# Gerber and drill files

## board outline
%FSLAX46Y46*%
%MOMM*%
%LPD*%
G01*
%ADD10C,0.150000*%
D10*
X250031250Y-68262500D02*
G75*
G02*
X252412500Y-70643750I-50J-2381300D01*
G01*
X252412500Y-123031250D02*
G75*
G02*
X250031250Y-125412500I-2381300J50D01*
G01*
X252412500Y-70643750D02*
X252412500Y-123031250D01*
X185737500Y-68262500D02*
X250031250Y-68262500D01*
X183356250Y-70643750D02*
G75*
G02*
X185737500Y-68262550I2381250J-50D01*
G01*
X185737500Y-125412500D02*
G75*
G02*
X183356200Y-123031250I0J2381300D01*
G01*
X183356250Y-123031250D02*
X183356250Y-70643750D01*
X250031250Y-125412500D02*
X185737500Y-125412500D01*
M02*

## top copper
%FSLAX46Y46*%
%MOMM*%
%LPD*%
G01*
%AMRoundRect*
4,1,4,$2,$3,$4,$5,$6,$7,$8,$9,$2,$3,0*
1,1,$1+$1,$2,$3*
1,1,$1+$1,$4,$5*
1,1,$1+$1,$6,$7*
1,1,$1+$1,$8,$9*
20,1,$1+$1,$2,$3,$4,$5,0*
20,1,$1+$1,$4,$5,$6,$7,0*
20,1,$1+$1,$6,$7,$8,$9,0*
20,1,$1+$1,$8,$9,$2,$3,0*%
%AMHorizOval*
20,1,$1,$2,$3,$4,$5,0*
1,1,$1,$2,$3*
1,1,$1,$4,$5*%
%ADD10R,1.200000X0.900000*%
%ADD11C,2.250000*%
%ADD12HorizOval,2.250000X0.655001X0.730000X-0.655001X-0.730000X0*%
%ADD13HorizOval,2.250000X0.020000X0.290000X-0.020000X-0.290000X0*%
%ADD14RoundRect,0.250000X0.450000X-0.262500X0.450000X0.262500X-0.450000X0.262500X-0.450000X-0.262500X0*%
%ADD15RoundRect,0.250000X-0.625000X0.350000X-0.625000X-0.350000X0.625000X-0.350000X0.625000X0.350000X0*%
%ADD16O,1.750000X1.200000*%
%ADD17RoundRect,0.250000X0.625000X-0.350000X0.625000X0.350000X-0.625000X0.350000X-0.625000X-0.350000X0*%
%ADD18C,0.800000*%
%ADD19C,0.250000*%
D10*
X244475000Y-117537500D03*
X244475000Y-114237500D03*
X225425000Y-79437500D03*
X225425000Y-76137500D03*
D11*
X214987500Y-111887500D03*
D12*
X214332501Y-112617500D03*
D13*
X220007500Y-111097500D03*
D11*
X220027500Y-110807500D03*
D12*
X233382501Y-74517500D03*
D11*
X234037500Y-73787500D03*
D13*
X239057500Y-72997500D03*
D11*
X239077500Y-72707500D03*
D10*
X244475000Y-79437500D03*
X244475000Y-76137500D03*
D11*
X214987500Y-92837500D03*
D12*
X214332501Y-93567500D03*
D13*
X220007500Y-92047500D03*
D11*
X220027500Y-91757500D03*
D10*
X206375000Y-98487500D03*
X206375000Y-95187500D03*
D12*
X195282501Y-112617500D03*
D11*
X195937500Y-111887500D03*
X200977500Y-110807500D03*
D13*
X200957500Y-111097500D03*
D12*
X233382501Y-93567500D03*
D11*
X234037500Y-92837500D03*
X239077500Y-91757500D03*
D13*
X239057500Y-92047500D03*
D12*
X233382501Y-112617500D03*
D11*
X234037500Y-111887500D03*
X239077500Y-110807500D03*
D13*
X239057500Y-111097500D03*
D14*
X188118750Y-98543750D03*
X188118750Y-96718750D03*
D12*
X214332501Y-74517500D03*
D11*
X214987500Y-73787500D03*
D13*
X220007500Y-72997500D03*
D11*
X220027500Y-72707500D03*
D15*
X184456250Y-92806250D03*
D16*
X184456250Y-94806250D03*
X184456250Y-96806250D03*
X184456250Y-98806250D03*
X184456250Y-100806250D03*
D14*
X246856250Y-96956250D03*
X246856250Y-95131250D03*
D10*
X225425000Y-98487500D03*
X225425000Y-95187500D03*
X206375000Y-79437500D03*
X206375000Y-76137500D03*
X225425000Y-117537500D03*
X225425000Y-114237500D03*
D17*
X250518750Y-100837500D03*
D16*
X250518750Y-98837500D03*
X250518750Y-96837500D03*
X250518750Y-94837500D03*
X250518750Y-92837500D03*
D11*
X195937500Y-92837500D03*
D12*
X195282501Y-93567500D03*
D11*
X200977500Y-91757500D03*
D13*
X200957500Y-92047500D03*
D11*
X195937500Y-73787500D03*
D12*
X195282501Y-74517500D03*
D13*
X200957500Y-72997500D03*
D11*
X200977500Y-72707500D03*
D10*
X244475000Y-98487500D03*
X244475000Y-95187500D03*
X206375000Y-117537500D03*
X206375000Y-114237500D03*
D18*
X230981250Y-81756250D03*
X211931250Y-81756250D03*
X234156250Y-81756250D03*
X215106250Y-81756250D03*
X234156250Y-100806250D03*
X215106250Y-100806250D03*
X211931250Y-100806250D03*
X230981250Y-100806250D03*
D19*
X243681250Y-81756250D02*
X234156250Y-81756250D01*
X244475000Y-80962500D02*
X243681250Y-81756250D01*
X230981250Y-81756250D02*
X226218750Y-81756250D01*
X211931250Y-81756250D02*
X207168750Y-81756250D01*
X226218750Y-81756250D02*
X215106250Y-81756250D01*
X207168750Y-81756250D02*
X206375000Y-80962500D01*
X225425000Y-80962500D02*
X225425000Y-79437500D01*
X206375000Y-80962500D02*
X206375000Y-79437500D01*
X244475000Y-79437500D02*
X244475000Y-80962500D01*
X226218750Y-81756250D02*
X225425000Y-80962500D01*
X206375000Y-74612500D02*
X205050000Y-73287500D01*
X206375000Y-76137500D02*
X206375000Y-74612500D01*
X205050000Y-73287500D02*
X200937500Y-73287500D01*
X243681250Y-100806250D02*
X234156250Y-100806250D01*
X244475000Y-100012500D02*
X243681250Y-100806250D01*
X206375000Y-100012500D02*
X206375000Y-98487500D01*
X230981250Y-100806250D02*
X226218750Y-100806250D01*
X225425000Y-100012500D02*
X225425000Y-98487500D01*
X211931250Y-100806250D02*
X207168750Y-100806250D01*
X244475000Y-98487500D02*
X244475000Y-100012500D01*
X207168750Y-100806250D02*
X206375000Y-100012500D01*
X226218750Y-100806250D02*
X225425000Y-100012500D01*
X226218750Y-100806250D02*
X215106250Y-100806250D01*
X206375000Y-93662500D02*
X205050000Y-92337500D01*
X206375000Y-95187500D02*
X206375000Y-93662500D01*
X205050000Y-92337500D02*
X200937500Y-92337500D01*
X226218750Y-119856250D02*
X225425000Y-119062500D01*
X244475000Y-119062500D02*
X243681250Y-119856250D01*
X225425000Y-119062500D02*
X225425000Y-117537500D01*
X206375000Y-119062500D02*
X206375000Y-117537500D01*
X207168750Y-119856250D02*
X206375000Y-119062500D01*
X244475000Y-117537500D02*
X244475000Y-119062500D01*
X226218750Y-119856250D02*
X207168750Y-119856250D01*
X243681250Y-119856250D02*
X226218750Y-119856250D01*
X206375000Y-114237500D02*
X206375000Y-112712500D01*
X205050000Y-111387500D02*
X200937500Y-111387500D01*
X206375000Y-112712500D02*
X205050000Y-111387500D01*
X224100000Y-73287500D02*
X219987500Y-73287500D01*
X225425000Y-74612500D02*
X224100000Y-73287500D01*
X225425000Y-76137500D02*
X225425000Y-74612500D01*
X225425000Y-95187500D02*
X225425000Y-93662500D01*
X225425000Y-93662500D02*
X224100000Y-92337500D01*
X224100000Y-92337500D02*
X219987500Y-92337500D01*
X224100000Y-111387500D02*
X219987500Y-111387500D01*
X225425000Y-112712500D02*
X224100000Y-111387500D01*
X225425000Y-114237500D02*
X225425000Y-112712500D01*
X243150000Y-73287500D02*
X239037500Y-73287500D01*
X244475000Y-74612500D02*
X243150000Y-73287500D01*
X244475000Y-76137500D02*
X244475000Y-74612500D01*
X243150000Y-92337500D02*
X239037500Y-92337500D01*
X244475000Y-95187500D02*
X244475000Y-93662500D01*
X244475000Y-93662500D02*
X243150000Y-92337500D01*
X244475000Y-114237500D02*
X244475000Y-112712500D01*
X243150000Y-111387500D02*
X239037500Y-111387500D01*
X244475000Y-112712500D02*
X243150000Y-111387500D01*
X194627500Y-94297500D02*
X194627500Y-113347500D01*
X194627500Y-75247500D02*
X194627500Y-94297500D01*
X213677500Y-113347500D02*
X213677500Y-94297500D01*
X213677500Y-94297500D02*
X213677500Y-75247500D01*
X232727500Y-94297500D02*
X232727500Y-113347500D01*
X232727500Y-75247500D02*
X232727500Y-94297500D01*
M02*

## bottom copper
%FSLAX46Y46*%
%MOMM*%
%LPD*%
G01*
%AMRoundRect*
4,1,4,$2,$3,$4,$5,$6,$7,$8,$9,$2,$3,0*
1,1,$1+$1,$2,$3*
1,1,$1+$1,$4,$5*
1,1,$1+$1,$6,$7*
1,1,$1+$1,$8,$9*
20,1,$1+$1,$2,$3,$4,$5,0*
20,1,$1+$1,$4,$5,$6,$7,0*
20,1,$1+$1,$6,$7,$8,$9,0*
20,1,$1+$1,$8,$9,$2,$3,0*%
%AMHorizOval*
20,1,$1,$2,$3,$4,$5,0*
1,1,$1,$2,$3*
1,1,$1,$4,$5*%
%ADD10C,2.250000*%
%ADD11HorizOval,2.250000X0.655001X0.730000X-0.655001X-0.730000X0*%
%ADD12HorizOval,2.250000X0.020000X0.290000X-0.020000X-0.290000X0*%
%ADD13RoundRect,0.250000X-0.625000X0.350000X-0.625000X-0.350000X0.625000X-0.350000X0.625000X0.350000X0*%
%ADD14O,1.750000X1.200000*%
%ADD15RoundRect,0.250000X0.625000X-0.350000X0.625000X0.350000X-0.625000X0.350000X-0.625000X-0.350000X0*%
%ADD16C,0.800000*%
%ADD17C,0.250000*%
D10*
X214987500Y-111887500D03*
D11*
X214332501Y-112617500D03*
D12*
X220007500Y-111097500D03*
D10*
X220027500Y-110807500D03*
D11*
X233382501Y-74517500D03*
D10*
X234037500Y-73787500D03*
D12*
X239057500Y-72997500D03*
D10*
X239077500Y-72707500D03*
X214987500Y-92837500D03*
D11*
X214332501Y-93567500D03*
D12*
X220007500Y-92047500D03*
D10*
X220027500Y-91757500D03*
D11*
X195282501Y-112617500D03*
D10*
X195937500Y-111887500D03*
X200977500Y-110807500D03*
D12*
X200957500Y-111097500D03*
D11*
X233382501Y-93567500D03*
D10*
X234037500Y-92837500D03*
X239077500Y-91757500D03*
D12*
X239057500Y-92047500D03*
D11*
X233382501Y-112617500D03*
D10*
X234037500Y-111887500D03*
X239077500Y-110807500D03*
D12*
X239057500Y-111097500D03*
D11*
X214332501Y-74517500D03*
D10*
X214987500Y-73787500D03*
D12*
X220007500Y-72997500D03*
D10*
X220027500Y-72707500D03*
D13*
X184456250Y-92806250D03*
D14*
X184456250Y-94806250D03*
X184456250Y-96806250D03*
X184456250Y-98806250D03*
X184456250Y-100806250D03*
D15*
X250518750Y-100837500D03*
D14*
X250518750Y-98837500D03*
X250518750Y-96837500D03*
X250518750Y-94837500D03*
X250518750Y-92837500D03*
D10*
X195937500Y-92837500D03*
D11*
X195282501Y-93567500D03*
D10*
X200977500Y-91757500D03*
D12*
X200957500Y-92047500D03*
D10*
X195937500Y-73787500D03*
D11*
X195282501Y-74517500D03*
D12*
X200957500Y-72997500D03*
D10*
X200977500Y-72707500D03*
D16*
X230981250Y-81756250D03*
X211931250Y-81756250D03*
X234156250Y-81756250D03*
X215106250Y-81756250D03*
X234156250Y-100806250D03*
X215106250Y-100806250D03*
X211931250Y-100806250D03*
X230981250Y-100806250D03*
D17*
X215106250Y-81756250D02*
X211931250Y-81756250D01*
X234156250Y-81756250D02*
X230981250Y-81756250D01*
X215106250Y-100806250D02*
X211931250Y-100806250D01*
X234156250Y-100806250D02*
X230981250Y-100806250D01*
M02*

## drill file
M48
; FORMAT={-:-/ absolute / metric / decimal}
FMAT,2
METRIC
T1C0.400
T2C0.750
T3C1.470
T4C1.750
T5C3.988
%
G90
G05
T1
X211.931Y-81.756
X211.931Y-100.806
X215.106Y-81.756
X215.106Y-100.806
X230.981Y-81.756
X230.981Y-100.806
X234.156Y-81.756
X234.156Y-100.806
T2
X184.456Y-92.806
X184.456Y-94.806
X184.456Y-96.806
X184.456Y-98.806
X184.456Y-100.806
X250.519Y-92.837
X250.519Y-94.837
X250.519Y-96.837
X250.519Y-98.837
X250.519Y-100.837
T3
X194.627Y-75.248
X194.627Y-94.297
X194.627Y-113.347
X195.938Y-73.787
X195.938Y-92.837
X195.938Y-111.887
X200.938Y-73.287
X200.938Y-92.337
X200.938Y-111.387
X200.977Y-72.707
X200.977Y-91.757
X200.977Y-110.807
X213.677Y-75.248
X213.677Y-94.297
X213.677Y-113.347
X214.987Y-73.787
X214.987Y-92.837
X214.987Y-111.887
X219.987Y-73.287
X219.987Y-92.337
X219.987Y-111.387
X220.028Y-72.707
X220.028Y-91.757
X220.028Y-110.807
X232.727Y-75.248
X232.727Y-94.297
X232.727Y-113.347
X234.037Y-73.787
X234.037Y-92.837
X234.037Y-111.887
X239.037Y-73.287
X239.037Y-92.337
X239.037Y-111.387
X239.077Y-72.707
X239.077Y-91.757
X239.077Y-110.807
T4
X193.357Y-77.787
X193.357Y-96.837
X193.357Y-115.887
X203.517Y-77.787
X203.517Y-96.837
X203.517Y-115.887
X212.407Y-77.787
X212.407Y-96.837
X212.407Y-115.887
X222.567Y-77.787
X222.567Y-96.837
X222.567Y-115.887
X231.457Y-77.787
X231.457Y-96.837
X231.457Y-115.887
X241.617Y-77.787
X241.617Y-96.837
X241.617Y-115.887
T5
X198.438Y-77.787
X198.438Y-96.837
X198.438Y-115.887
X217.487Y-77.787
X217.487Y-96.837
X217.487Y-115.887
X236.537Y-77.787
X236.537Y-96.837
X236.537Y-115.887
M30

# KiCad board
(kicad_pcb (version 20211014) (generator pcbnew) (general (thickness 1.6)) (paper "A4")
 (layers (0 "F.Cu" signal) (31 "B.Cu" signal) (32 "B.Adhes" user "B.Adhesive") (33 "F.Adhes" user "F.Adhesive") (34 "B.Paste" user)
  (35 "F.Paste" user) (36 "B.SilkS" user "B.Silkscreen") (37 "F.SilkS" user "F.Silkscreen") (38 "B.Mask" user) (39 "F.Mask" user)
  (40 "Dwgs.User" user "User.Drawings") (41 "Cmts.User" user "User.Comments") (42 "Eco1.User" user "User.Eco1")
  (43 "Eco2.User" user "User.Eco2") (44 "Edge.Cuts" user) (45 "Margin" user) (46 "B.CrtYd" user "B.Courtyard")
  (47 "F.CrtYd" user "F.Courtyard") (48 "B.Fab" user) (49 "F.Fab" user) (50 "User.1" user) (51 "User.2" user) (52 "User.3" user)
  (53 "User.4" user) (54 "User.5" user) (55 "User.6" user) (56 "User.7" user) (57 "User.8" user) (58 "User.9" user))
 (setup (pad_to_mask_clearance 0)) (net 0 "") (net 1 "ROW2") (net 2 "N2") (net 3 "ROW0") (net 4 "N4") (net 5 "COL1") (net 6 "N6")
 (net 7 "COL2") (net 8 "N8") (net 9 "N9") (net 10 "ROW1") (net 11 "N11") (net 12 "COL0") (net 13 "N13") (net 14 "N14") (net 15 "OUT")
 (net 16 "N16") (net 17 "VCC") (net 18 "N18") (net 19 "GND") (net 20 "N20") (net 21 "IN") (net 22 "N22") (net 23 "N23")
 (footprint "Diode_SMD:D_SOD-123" (layer "F.Cu") (at 244.475 115.8875 90)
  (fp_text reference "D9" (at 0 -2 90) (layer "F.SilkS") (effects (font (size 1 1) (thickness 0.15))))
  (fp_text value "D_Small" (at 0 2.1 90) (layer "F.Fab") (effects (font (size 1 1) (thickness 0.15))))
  (pad "1" smd rect (at -1.65 0 90) (size 0.9 1.2) (layers "F.Cu" "F.Paste" "F.Mask") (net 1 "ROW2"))
  (pad "2" smd rect (at 1.65 0 90) (size 0.9 1.2) (layers "F.Cu" "F.Paste" "F.Mask") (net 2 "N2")))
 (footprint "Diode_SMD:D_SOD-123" (layer "F.Cu") (at 225.425 77.7875 90)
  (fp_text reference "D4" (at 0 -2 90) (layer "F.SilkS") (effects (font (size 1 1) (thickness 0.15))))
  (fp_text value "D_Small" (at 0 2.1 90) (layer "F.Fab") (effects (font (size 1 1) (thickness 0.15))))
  (pad "1" smd rect (at -1.65 0 90) (size 0.9 1.2) (layers "F.Cu" "F.Paste" "F.Mask") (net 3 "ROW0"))
  (pad "2" smd rect (at 1.65 0 90) (size 0.9 1.2) (layers "F.Cu" "F.Paste" "F.Mask") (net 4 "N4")))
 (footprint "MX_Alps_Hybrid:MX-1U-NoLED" (layer "F.Cu") (at 217.4875 115.8875)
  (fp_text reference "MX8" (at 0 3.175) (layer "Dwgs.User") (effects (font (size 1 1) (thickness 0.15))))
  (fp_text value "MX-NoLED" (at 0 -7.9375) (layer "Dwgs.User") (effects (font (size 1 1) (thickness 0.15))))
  (pad "" np_thru_hole circle locked (at -5.08 0 48.0996) (size 1.75 1.75) (drill 1.75) (layers *.Cu *.Mask))
  (pad "" np_thru_hole circle locked (at 0 0) (size 3.9878 3.9878) (drill 3.9878) (layers *.Cu *.Mask))
  (pad "" np_thru_hole circle locked (at 5.08 0 48.0996) (size 1.75 1.75) (drill 1.75) (layers *.Cu *.Mask))
  (pad "1" thru_hole circle locked (at -2.5 -4) (size 2.25 2.25) (drill 1.47) (layers *.Cu "B.Mask") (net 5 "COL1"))
  (pad "1" thru_hole oval locked (at -3.81 -2.54 48.0996) (size 4.211556 2.25) (drill 1.47 (offset 0.980778 0)) (layers *.Cu "B.Mask")
   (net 5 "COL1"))
  (pad "2" thru_hole oval locked (at 2.5 -4.5 86.0548) (size 2.831378 2.25) (drill 1.47 (offset 0.290689 0)) (layers *.Cu "B.Mask")
   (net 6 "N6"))
  (pad "2" thru_hole circle locked (at 2.54 -5.08) (size 2.25 2.25) (drill 1.47) (layers *.Cu "B.Mask") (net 6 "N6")))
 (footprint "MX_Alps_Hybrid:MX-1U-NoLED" (layer "F.Cu") (at 236.5375 77.7875)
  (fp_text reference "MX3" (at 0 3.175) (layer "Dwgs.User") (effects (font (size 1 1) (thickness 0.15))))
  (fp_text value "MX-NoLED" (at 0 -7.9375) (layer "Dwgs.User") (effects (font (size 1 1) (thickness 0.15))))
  (pad "" np_thru_hole circle locked (at -5.08 0 48.0996) (size 1.75 1.75) (drill 1.75) (layers *.Cu *.Mask))
  (pad "" np_thru_hole circle locked (at 0 0) (size 3.9878 3.9878) (drill 3.9878) (layers *.Cu *.Mask))
  (pad "" np_thru_hole circle locked (at 5.08 0 48.0996) (size 1.75 1.75) (drill 1.75) (layers *.Cu *.Mask))
  (pad "1" thru_hole oval locked (at -3.81 -2.54 48.0996) (size 4.211556 2.25) (drill 1.47 (offset 0.980778 0)) (layers *.Cu "B.Mask")
   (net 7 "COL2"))
  (pad "1" thru_hole circle locked (at -2.5 -4) (size 2.25 2.25) (drill 1.47) (layers *.Cu "B.Mask") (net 7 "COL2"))
  (pad "2" thru_hole oval locked (at 2.5 -4.5 86.0548) (size 2.831378 2.25) (drill 1.47 (offset 0.290689 0)) (layers *.Cu "B.Mask")
   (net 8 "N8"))
  (pad "2" thru_hole circle locked (at 2.54 -5.08) (size 2.25 2.25) (drill 1.47) (layers *.Cu "B.Mask") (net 8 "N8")))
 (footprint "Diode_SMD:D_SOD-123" (layer "F.Cu") (at 244.475 77.7875 90)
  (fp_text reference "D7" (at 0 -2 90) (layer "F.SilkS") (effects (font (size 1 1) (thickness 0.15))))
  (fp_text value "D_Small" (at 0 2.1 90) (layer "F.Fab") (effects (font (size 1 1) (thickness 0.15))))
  (pad "1" smd rect (at -1.65 0 90) (size 0.9 1.2) (layers "F.Cu" "F.Paste" "F.Mask") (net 3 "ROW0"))
  (pad "2" smd rect (at 1.65 0 90) (size 0.9 1.2) (layers "F.Cu" "F.Paste" "F.Mask") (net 8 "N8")))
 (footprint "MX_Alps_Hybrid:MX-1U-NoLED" (layer "F.Cu") (at 217.4875 96.8375)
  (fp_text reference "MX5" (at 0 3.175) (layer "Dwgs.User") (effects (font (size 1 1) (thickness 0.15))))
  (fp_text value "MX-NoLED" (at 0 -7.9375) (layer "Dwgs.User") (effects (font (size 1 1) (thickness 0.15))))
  (pad "" np_thru_hole circle locked (at -5.08 0 48.0996) (size 1.75 1.75) (drill 1.75) (layers *.Cu *.Mask))
  (pad "" np_thru_hole circle locked (at 0 0) (size 3.9878 3.9878) (drill 3.9878) (layers *.Cu *.Mask))
  (pad "" np_thru_hole circle locked (at 5.08 0 48.0996) (size 1.75 1.75) (drill 1.75) (layers *.Cu *.Mask))
  (pad "1" thru_hole circle locked (at -2.5 -4) (size 2.25 2.25) (drill 1.47) (layers *.Cu "B.Mask") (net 5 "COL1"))
  (pad "1" thru_hole oval locked (at -3.81 -2.54 48.0996) (size 4.211556 2.25) (drill 1.47 (offset 0.980778 0)) (layers *.Cu "B.Mask")
   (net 5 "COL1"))
  (pad "2" thru_hole oval locked (at 2.5 -4.5 86.0548) (size 2.831378 2.25) (drill 1.47 (offset 0.290689 0)) (layers *.Cu "B.Mask")
   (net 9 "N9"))
  (pad "2" thru_hole circle locked (at 2.54 -5.08) (size 2.25 2.25) (drill 1.47) (layers *.Cu "B.Mask") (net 9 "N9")))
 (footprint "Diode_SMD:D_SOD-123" (layer "F.Cu") (at 206.375 96.8375 90)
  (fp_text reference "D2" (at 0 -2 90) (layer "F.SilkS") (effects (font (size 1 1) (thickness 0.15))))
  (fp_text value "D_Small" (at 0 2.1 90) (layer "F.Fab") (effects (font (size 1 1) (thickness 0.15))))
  (pad "1" smd rect (at -1.65 0 90) (size 0.9 1.2) (layers "F.Cu" "F.Paste" "F.Mask") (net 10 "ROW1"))
  (pad "2" smd rect (at 1.65 0 90) (size 0.9 1.2) (layers "F.Cu" "F.Paste" "F.Mask") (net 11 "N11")))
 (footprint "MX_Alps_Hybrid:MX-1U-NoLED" (layer "F.Cu") (at 198.4375 115.8875)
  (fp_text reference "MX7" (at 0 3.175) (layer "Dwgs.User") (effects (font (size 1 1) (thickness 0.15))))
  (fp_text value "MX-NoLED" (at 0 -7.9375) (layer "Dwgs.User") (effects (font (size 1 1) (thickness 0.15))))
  (pad "" np_thru_hole circle locked (at 0 0) (size 3.9878 3.9878) (drill 3.9878) (layers *.Cu *.Mask))
  (pad "" np_thru_hole circle locked (at -5.08 0 48.0996) (size 1.75 1.75) (drill 1.75) (layers *.Cu *.Mask))
  (pad "" np_thru_hole circle locked (at 5.08 0 48.0996) (size 1.75 1.75) (drill 1.75) (layers *.Cu *.Mask))
  (pad "1" thru_hole oval locked (at -3.81 -2.54 48.0996) (size 4.211556 2.25) (drill 1.47 (offset 0.980778 0)) (layers *.Cu "B.Mask")
   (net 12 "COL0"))
  (pad "1" thru_hole circle locked (at -2.5 -4) (size 2.25 2.25) (drill 1.47) (layers *.Cu "B.Mask") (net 12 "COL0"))
  (pad "2" thru_hole circle locked (at 2.54 -5.08) (size 2.25 2.25) (drill 1.47) (layers *.Cu "B.Mask") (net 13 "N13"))
  (pad "2" thru_hole oval locked (at 2.5 -4.5 86.0548) (size 2.831378 2.25) (drill 1.47 (offset 0.290689 0)) (layers *.Cu "B.Mask")
   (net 13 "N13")))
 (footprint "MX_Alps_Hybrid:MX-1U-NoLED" (layer "F.Cu") (at 236.5375 96.8375)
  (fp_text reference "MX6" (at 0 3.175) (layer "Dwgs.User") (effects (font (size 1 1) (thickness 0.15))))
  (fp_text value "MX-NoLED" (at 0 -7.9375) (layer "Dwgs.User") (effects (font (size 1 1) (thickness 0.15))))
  (pad "" np_thru_hole circle locked (at 5.08 0 48.0996) (size 1.75 1.75) (drill 1.75) (layers *.Cu *.Mask))
  (pad "" np_thru_hole circle locked (at -5.08 0 48.0996) (size 1.75 1.75) (drill 1.75) (layers *.Cu *.Mask))
  (pad "" np_thru_hole circle locked (at 0 0) (size 3.9878 3.9878) (drill 3.9878) (layers *.Cu *.Mask))
  (pad "1" thru_hole oval locked (at -3.81 -2.54 48.0996) (size 4.211556 2.25) (drill 1.47 (offset 0.980778 0)) (layers *.Cu "B.Mask")
   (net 7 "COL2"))
  (pad "1" thru_hole circle locked (at -2.5 -4) (size 2.25 2.25) (drill 1.47) (layers *.Cu "B.Mask") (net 7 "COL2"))
  (pad "2" thru_hole circle locked (at 2.54 -5.08) (size 2.25 2.25) (drill 1.47) (layers *.Cu "B.Mask") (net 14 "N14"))
  (pad "2" thru_hole oval locked (at 2.5 -4.5 86.0548) (size 2.831378 2.25) (drill 1.47 (offset 0.290689 0)) (layers *.Cu "B.Mask")
   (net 14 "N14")))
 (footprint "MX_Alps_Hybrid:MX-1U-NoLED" (layer "F.Cu") (at 236.5375 115.8875)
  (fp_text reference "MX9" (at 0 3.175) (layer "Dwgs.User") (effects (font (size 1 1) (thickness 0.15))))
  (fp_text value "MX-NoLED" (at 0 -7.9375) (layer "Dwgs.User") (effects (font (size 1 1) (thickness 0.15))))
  (pad "" np_thru_hole circle locked (at -5.08 0 48.0996) (size 1.75 1.75) (drill 1.75) (layers *.Cu *.Mask))
  (pad "" np_thru_hole circle locked (at 5.08 0 48.0996) (size 1.75 1.75) (drill 1.75) (layers *.Cu *.Mask))
  (pad "" np_thru_hole circle locked (at 0 0) (size 3.9878 3.9878) (drill 3.9878) (layers *.Cu *.Mask))
  (pad "1" thru_hole oval locked (at -3.81 -2.54 48.0996) (size 4.211556 2.25) (drill 1.47 (offset 0.980778 0)) (layers *.Cu "B.Mask")
   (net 7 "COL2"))
  (pad "1" thru_hole circle locked (at -2.5 -4) (size 2.25 2.25) (drill 1.47) (layers *.Cu "B.Mask") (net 7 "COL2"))
  (pad "2" thru_hole circle locked (at 2.54 -5.08) (size 2.25 2.25) (drill 1.47) (layers *.Cu "B.Mask") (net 2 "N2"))
  (pad "2" thru_hole oval locked (at 2.5 -4.5 86.0548) (size 2.831378 2.25) (drill 1.47 (offset 0.290689 0)) (layers *.Cu "B.Mask")
   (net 2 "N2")))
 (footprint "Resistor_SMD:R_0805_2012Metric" (layer "F.Cu") (at 188.11875 97.63125 90)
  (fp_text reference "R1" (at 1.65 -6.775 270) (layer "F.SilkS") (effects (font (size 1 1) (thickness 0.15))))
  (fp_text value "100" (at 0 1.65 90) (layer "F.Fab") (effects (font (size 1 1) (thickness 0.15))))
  (pad "1" smd roundrect (at -0.9125 0 90) (size 1.025 1.4) (layers "F.Cu" "F.Paste" "F.Mask") (roundrect_rratio 0.243902) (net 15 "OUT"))
  (pad "2" smd roundrect (at 0.9125 0 90) (size 1.025 1.4) (layers "F.Cu" "F.Paste" "F.Mask") (roundrect_rratio 0.243902) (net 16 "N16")))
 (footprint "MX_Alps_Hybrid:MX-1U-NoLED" (layer "F.Cu") (at 217.4875 77.7875)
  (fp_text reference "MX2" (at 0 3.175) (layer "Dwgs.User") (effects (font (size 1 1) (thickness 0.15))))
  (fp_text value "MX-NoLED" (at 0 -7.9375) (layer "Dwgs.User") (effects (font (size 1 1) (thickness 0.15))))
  (pad "" np_thru_hole circle locked (at -5.08 0 48.0996) (size 1.75 1.75) (drill 1.75) (layers *.Cu *.Mask))
  (pad "" np_thru_hole circle locked (at 5.08 0 48.0996) (size 1.75 1.75) (drill 1.75) (layers *.Cu *.Mask))
  (pad "" np_thru_hole circle locked (at 0 0) (size 3.9878 3.9878) (drill 3.9878) (layers *.Cu *.Mask))
  (pad "1" thru_hole oval locked (at -3.81 -2.54 48.0996) (size 4.211556 2.25) (drill 1.47 (offset 0.980778 0)) (layers *.Cu "B.Mask")
   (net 5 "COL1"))
  (pad "1" thru_hole circle locked (at -2.5 -4) (size 2.25 2.25) (drill 1.47) (layers *.Cu "B.Mask") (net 5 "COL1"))
  (pad "2" thru_hole oval locked (at 2.5 -4.5 86.0548) (size 2.831378 2.25) (drill 1.47 (offset 0.290689 0)) (layers *.Cu "B.Mask")
   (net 4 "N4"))
  (pad "2" thru_hole circle locked (at 2.54 -5.08) (size 2.25 2.25) (drill 1.47) (layers *.Cu "B.Mask") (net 4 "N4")))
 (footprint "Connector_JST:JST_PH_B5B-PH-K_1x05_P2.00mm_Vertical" (layer "F.Cu") (at 184.45625 92.80625 -90)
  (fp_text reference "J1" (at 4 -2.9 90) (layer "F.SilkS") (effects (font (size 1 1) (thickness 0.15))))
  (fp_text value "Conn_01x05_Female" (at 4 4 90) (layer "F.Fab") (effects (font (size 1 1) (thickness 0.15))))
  (pad "1" thru_hole roundrect (at 0 0 270) (size 1.2 1.75) (drill 0.75) (layers *.Cu *.Mask) (roundrect_rratio 0.208333) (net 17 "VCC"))
  (pad "2" thru_hole oval (at 2 0 270) (size 1.2 1.75) (drill 0.75) (layers *.Cu *.Mask) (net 17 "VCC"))
  (pad "3" thru_hole oval (at 4 0 270) (size 1.2 1.75) (drill 0.75) (layers *.Cu *.Mask) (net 16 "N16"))
  (pad "4" thru_hole oval (at 6 0 270) (size 1.2 1.75) (drill 0.75) (layers *.Cu *.Mask) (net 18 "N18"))
  (pad "5" thru_hole oval (at 8 0 270) (size 1.2 1.75) (drill 0.75) (layers *.Cu *.Mask) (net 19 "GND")))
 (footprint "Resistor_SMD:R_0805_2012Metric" (layer "F.Cu") (at 246.85625 96.04375 90)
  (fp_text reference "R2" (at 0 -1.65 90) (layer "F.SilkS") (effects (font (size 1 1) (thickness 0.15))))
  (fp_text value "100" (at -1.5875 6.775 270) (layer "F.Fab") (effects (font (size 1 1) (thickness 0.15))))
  (pad "1" smd roundrect (at -0.9125 0 90) (size 1.025 1.4) (layers "F.Cu" "F.Paste" "F.Mask") (roundrect_rratio 0.243902) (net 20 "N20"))
  (pad "2" smd roundrect (at 0.9125 0 90) (size 1.025 1.4) (layers "F.Cu" "F.Paste" "F.Mask") (roundrect_rratio 0.243902) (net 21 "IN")))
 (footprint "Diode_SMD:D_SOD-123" (layer "F.Cu") (at 225.425 96.8375 90)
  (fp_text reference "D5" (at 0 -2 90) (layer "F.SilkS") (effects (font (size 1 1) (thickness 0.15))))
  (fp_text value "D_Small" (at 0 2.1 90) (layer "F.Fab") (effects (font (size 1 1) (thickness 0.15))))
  (pad "1" smd rect (at -1.65 0 90) (size 0.9 1.2) (layers "F.Cu" "F.Paste" "F.Mask") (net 10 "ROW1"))
  (pad "2" smd rect (at 1.65 0 90) (size 0.9 1.2) (layers "F.Cu" "F.Paste" "F.Mask") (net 9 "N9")))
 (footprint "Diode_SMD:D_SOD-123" (layer "F.Cu") (at 206.375 77.7875 90)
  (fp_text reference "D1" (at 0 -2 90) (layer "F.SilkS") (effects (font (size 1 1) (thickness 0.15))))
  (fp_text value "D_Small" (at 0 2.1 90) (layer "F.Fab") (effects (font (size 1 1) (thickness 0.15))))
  (pad "1" smd rect (at -1.65 0 90) (size 0.9 1.2) (layers "F.Cu" "F.Paste" "F.Mask") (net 3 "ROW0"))
  (pad "2" smd rect (at 1.65 0 90) (size 0.9 1.2) (layers "F.Cu" "F.Paste" "F.Mask") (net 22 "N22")))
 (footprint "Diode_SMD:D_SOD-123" (layer "F.Cu") (at 225.425 115.8875 90)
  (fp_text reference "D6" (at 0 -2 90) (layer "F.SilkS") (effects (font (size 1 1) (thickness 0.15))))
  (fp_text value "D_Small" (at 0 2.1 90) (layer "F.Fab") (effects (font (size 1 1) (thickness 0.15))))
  (pad "1" smd rect (at -1.65 0 90) (size 0.9 1.2) (layers "F.Cu" "F.Paste" "F.Mask") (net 1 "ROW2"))
  (pad "2" smd rect (at 1.65 0 90) (size 0.9 1.2) (layers "F.Cu" "F.Paste" "F.Mask") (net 6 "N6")))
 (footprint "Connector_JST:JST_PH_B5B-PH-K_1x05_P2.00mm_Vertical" (layer "F.Cu") (at 250.51875 100.8375 90)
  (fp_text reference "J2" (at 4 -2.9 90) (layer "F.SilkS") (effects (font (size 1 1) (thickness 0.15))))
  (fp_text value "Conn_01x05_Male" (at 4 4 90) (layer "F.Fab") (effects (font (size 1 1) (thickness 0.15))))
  (pad "1" thru_hole roundrect (at 0 0 90) (size 1.2 1.75) (drill 0.75) (layers *.Cu *.Mask) (roundrect_rratio 0.208333) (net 17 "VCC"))
  (pad "2" thru_hole oval (at 2 0 90) (size 1.2 1.75) (drill 0.75) (layers *.Cu *.Mask) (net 17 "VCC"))
  (pad "3" thru_hole oval (at 4 0 90) (size 1.2 1.75) (drill 0.75) (layers *.Cu *.Mask) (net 20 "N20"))
  (pad "4" thru_hole oval (at 6 0 90) (size 1.2 1.75) (drill 0.75) (layers *.Cu *.Mask) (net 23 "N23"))
  (pad "5" thru_hole oval (at 8 0 90) (size 1.2 1.75) (drill 0.75) (layers *.Cu *.Mask) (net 19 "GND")))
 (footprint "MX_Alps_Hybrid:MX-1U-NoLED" (layer "F.Cu") (at 198.4375 96.8375)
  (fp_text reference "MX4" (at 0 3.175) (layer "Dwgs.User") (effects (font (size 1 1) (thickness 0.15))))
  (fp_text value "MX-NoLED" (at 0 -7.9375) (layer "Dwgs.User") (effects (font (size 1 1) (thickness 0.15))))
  (pad "" np_thru_hole circle locked (at -5.08 0 48.0996) (size 1.75 1.75) (drill 1.75) (layers *.Cu *.Mask))
  (pad "" np_thru_hole circle locked (at 5.08 0 48.0996) (size 1.75 1.75) (drill 1.75) (layers *.Cu *.Mask))
  (pad "" np_thru_hole circle locked (at 0 0) (size 3.9878 3.9878) (drill 3.9878) (layers *.Cu *.Mask))
  (pad "1" thru_hole circle locked (at -2.5 -4) (size 2.25 2.25) (drill 1.47) (layers *.Cu "B.Mask") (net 12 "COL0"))
  (pad "1" thru_hole oval locked (at -3.81 -2.54 48.0996) (size 4.211556 2.25) (drill 1.47 (offset 0.980778 0)) (layers *.Cu "B.Mask")
   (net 12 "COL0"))
  (pad "2" thru_hole circle locked (at 2.54 -5.08) (size 2.25 2.25) (drill 1.47) (layers *.Cu "B.Mask") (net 11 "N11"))
  (pad "2" thru_hole oval locked (at 2.5 -4.5 86.0548) (size 2.831378 2.25) (drill 1.47 (offset 0.290689 0)) (layers *.Cu "B.Mask")
   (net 11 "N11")))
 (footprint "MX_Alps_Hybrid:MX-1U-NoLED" (layer "F.Cu") (at 198.4375 77.7875)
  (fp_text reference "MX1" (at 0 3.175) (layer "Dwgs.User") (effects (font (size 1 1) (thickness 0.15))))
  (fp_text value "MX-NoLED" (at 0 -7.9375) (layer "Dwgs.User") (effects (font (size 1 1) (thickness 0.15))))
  (pad "" np_thru_hole circle locked (at 5.08 0 48.0996) (size 1.75 1.75) (drill 1.75) (layers *.Cu *.Mask))
  (pad "" np_thru_hole circle locked (at -5.08 0 48.0996) (size 1.75 1.75) (drill 1.75) (layers *.Cu *.Mask))
  (pad "" np_thru_hole circle locked (at 0 0) (size 3.9878 3.9878) (drill 3.9878) (layers *.Cu *.Mask))
  (pad "1" thru_hole circle locked (at -2.5 -4) (size 2.25 2.25) (drill 1.47) (layers *.Cu "B.Mask") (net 12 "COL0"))
  (pad "1" thru_hole oval locked (at -3.81 -2.54 48.0996) (size 4.211556 2.25) (drill 1.47 (offset 0.980778 0)) (layers *.Cu "B.Mask")
   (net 12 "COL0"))
  (pad "2" thru_hole oval locked (at 2.5 -4.5 86.0548) (size 2.831378 2.25) (drill 1.47 (offset 0.290689 0)) (layers *.Cu "B.Mask")
   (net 22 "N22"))
  (pad "2" thru_hole circle locked (at 2.54 -5.08) (size 2.25 2.25) (drill 1.47) (layers *.Cu "B.Mask") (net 22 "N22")))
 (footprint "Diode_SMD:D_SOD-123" (layer "F.Cu") (at 244.475 96.8375 90)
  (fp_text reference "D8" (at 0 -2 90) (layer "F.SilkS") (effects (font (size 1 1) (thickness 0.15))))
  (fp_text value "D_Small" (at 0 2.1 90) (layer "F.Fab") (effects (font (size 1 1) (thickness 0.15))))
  (pad "1" smd rect (at -1.65 0 90) (size 0.9 1.2) (layers "F.Cu" "F.Paste" "F.Mask") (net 10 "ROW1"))
  (pad "2" smd rect (at 1.65 0 90) (size 0.9 1.2) (layers "F.Cu" "F.Paste" "F.Mask") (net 14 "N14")))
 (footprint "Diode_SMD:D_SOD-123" (layer "F.Cu") (at 206.375 115.8875 90)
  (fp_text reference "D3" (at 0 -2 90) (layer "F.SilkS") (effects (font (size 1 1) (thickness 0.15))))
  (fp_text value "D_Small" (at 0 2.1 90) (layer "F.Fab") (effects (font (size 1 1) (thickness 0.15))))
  (pad "1" smd rect (at -1.65 0 90) (size 0.9 1.2) (layers "F.Cu" "F.Paste" "F.Mask") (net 1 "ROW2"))
  (pad "2" smd rect (at 1.65 0 90) (size 0.9 1.2) (layers "F.Cu" "F.Paste" "F.Mask") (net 13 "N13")))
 (gr_arc (start 250.03125 68.2625) (mid 251.715048 68.959952) (end 252.4125 70.64375) (layer "Edge.Cuts") (width 0.15))
 (gr_arc (start 252.4125 123.03125) (mid 251.715048 124.715048) (end 250.03125 125.4125) (layer "Edge.Cuts") (width 0.15))
 (gr_line (start 252.4125 70.64375) (end 252.4125 123.03125) (layer "Edge.Cuts") (width 0.15))
 (gr_line (start 185.7375 68.2625) (end 250.03125 68.2625) (layer "Edge.Cuts") (width 0.15))
 (gr_arc (start 183.35625 70.64375) (mid 184.053702 68.959952) (end 185.7375 68.2625) (layer "Edge.Cuts") (width 0.15))
 (gr_arc (start 185.7375 125.4125) (mid 184.053702 124.715048) (end 183.35625 123.03125) (layer "Edge.Cuts") (width 0.15))
 (gr_line (start 183.35625 123.03125) (end 183.35625 70.64375) (layer "Edge.Cuts") (width 0.15))
 (gr_line (start 250.03125 125.4125) (end 185.7375 125.4125) (layer "Edge.Cuts") (width 0.15))
 (segment (start 243.68125 81.75625) (end 234.15625 81.75625) (width 0.25) (layer "F.Cu") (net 3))
 (segment (start 244.475 80.9625) (end 243.68125 81.75625) (width 0.25) (layer "F.Cu") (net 3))
 (segment (start 230.98125 81.75625) (end 226.21875 81.75625) (width 0.25) (layer "F.Cu") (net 3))
 (segment (start 211.93125 81.75625) (end 207.16875 81.75625) (width 0.25) (layer "F.Cu") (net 3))
 (segment (start 226.21875 81.75625) (end 215.10625 81.75625) (width 0.25) (layer "F.Cu") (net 3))
 (segment (start 207.16875 81.75625) (end 206.375 80.9625) (width 0.25) (layer "F.Cu") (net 3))
 (segment (start 225.425 80.9625) (end 225.425 79.4375) (width 0.25) (layer "F.Cu") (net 3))
 (segment (start 206.375 80.9625) (end 206.375 79.4375) (width 0.25) (layer "F.Cu") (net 3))
 (segment (start 244.475 79.4375) (end 244.475 80.9625) (width 0.25) (layer "F.Cu") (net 3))
 (segment (start 226.21875 81.75625) (end 225.425 80.9625) (width 0.25) (layer "F.Cu") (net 3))
 (via (at 230.98125 81.75625) (size 0.8) (drill 0.4) (layers "F.Cu" "B.Cu") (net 3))
 (via (at 211.93125 81.75625) (size 0.8) (drill 0.4) (layers "F.Cu" "B.Cu") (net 3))
 (via (at 234.15625 81.75625) (size 0.8) (drill 0.4) (layers "F.Cu" "B.Cu") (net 3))
 (via (at 215.10625 81.75625) (size 0.8) (drill 0.4) (layers "F.Cu" "B.Cu") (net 3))
 (segment (start 215.10625 81.75625) (end 211.93125 81.75625) (width 0.25) (layer "B.Cu") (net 3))
 (segment (start 234.15625 81.75625) (end 230.98125 81.75625) (width 0.25) (layer "B.Cu") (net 3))
 (segment (start 206.375 74.6125) (end 205.05 73.2875) (width 0.25) (layer "F.Cu") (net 22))
 (segment (start 206.375 76.1375) (end 206.375 74.6125) (width 0.25) (layer "F.Cu") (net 22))
 (segment (start 205.05 73.2875) (end 200.9375 73.2875) (width 0.25) (layer "F.Cu") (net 22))
 (segment (start 243.68125 100.80625) (end 234.15625 100.80625) (width 0.25) (layer "F.Cu") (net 10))
 (segment (start 244.475 100.0125) (end 243.68125 100.80625) (width 0.25) (layer "F.Cu") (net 10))
 (segment (start 206.375 100.0125) (end 206.375 98.4875) (width 0.25) (layer "F.Cu") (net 10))
 (segment (start 230.98125 100.80625) (end 226.21875 100.80625) (width 0.25) (layer "F.Cu") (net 10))
 (segment (start 225.425 100.0125) (end 225.425 98.4875) (width 0.25) (layer "F.Cu") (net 10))
 (segment (start 211.93125 100.80625) (end 207.16875 100.80625) (width 0.25) (layer "F.Cu") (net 10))
 (segment (start 244.475 98.4875) (end 244.475 100.0125) (width 0.25) (layer "F.Cu") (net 10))
 (segment (start 207.16875 100.80625) (end 206.375 100.0125) (width 0.25) (layer "F.Cu") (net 10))
 (segment (start 226.21875 100.80625) (end 225.425 100.0125) (width 0.25) (layer "F.Cu") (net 10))
 (segment (start 226.21875 100.80625) (end 215.10625 100.80625) (width 0.25) (layer "F.Cu") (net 10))
 (via (at 234.15625 100.80625) (size 0.8) (drill 0.4) (layers "F.Cu" "B.Cu") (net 10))
 (via (at 215.10625 100.80625) (size 0.8) (drill 0.4) (layers "F.Cu" "B.Cu") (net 10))
 (via (at 211.93125 100.80625) (size 0.8) (drill 0.4) (layers "F.Cu" "B.Cu") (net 10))
 (via (at 230.98125 100.80625) (size 0.8) (drill 0.4) (layers "F.Cu" "B.Cu") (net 10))
 (segment (start 215.10625 100.80625) (end 211.93125 100.80625) (width 0.25) (layer "B.Cu") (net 10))
 (segment (start 234.15625 100.80625) (end 230.98125 100.80625) (width 0.25) (layer "B.Cu") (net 10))
 (segment (start 206.375 93.6625) (end 205.05 92.3375) (width 0.25) (layer "F.Cu") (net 11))
 (segment (start 206.375 95.1875) (end 206.375 93.6625) (width 0.25) (layer "F.Cu") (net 11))
 (segment (start 205.05 92.3375) (end 200.9375 92.3375) (width 0.25) (layer "F.Cu") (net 11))
 (segment (start 226.21875 119.85625) (end 225.425 119.0625) (width 0.25) (layer "F.Cu") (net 1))
 (segment (start 244.475 119.0625) (end 243.68125 119.85625) (width 0.25) (layer "F.Cu") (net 1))
 (segment (start 225.425 119.0625) (end 225.425 117.5375) (width 0.25) (layer "F.Cu") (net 1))
 (segment (start 206.375 119.0625) (end 206.375 117.5375) (width 0.25) (layer "F.Cu") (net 1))
 (segment (start 207.16875 119.85625) (end 206.375 119.0625) (width 0.25) (layer "F.Cu") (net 1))
 (segment (start 244.475 117.5375) (end 244.475 119.0625) (width 0.25) (layer "F.Cu") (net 1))
 (segment (start 226.21875 119.85625) (end 207.16875 119.85625) (width 0.25) (layer "F.Cu") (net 1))
 (segment (start 243.68125 119.85625) (end 226.21875 119.85625) (width 0.25) (layer "F.Cu") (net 1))
 (segment (start 206.375 114.2375) (end 206.375 112.7125) (width 0.25) (layer "F.Cu") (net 13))
 (segment (start 205.05 111.3875) (end 200.9375 111.3875) (width 0.25) (layer "F.Cu") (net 13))
 (segment (start 206.375 112.7125) (end 205.05 111.3875) (width 0.25) (layer "F.Cu") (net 13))
 (segment (start 224.1 73.2875) (end 219.9875 73.2875) (width 0.25) (layer "F.Cu") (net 4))
 (segment (start 225.425 74.6125) (end 224.1 73.2875) (width 0.25) (layer "F.Cu") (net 4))
 (segment (start 225.425 76.1375) (end 225.425 74.6125) (width 0.25) (layer "F.Cu") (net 4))
 (segment (start 225.425 95.1875) (end 225.425 93.6625) (width 0.25) (layer "F.Cu") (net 9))
 (segment (start 225.425 93.6625) (end 224.1 92.3375) (width 0.25) (layer "F.Cu") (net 9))
 (segment (start 224.1 92.3375) (end 219.9875 92.3375) (width 0.25) (layer "F.Cu") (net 9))
 (segment (start 224.1 111.3875) (end 219.9875 111.3875) (width 0.25) (layer "F.Cu") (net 6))
 (segment (start 225.425 112.7125) (end 224.1 111.3875) (width 0.25) (layer "F.Cu") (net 6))
 (segment (start 225.425 114.2375) (end 225.425 112.7125) (width 0.25) (layer "F.Cu") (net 6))
 (segment (start 243.15 73.2875) (end 239.0375 73.2875) (width 0.25) (layer "F.Cu") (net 8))
 (segment (start 244.475 74.6125) (end 243.15 73.2875) (width 0.25) (layer "F.Cu") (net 8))
 (segment (start 244.475 76.1375) (end 244.475 74.6125) (width 0.25) (layer "F.Cu") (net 8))
 (segment (start 243.15 92.3375) (end 239.0375 92.3375) (width 0.25) (layer "F.Cu") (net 14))
 (segment (start 244.475 95.1875) (end 244.475 93.6625) (width 0.25) (layer "F.Cu") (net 14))
 (segment (start 244.475 93.6625) (end 243.15 92.3375) (width 0.25) (layer "F.Cu") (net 14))
 (segment (start 244.475 114.2375) (end 244.475 112.7125) (width 0.25) (layer "F.Cu") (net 2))
 (segment (start 243.15 111.3875) (end 239.0375 111.3875) (width 0.25) (layer "F.Cu") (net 2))
 (segment (start 244.475 112.7125) (end 243.15 111.3875) (width 0.25) (layer "F.Cu") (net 2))
 (segment (start 194.6275 94.2975) (end 194.6275 113.3475) (width 0.25) (layer "F.Cu") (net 12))
 (segment (start 194.6275 75.2475) (end 194.6275 94.2975) (width 0.25) (layer "F.Cu") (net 12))
 (segment (start 213.6775 113.3475) (end 213.6775 94.2975) (width 0.25) (layer "F.Cu") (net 5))
 (segment (start 213.6775 94.2975) (end 213.6775 75.2475) (width 0.25) (layer "F.Cu") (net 5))
 (segment (start 232.7275 94.2975) (end 232.7275 113.3475) (width 0.25) (layer "F.Cu") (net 7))
 (segment (start 232.7275 75.2475) (end 232.7275 94.2975) (width 0.25) (layer "F.Cu") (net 7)))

